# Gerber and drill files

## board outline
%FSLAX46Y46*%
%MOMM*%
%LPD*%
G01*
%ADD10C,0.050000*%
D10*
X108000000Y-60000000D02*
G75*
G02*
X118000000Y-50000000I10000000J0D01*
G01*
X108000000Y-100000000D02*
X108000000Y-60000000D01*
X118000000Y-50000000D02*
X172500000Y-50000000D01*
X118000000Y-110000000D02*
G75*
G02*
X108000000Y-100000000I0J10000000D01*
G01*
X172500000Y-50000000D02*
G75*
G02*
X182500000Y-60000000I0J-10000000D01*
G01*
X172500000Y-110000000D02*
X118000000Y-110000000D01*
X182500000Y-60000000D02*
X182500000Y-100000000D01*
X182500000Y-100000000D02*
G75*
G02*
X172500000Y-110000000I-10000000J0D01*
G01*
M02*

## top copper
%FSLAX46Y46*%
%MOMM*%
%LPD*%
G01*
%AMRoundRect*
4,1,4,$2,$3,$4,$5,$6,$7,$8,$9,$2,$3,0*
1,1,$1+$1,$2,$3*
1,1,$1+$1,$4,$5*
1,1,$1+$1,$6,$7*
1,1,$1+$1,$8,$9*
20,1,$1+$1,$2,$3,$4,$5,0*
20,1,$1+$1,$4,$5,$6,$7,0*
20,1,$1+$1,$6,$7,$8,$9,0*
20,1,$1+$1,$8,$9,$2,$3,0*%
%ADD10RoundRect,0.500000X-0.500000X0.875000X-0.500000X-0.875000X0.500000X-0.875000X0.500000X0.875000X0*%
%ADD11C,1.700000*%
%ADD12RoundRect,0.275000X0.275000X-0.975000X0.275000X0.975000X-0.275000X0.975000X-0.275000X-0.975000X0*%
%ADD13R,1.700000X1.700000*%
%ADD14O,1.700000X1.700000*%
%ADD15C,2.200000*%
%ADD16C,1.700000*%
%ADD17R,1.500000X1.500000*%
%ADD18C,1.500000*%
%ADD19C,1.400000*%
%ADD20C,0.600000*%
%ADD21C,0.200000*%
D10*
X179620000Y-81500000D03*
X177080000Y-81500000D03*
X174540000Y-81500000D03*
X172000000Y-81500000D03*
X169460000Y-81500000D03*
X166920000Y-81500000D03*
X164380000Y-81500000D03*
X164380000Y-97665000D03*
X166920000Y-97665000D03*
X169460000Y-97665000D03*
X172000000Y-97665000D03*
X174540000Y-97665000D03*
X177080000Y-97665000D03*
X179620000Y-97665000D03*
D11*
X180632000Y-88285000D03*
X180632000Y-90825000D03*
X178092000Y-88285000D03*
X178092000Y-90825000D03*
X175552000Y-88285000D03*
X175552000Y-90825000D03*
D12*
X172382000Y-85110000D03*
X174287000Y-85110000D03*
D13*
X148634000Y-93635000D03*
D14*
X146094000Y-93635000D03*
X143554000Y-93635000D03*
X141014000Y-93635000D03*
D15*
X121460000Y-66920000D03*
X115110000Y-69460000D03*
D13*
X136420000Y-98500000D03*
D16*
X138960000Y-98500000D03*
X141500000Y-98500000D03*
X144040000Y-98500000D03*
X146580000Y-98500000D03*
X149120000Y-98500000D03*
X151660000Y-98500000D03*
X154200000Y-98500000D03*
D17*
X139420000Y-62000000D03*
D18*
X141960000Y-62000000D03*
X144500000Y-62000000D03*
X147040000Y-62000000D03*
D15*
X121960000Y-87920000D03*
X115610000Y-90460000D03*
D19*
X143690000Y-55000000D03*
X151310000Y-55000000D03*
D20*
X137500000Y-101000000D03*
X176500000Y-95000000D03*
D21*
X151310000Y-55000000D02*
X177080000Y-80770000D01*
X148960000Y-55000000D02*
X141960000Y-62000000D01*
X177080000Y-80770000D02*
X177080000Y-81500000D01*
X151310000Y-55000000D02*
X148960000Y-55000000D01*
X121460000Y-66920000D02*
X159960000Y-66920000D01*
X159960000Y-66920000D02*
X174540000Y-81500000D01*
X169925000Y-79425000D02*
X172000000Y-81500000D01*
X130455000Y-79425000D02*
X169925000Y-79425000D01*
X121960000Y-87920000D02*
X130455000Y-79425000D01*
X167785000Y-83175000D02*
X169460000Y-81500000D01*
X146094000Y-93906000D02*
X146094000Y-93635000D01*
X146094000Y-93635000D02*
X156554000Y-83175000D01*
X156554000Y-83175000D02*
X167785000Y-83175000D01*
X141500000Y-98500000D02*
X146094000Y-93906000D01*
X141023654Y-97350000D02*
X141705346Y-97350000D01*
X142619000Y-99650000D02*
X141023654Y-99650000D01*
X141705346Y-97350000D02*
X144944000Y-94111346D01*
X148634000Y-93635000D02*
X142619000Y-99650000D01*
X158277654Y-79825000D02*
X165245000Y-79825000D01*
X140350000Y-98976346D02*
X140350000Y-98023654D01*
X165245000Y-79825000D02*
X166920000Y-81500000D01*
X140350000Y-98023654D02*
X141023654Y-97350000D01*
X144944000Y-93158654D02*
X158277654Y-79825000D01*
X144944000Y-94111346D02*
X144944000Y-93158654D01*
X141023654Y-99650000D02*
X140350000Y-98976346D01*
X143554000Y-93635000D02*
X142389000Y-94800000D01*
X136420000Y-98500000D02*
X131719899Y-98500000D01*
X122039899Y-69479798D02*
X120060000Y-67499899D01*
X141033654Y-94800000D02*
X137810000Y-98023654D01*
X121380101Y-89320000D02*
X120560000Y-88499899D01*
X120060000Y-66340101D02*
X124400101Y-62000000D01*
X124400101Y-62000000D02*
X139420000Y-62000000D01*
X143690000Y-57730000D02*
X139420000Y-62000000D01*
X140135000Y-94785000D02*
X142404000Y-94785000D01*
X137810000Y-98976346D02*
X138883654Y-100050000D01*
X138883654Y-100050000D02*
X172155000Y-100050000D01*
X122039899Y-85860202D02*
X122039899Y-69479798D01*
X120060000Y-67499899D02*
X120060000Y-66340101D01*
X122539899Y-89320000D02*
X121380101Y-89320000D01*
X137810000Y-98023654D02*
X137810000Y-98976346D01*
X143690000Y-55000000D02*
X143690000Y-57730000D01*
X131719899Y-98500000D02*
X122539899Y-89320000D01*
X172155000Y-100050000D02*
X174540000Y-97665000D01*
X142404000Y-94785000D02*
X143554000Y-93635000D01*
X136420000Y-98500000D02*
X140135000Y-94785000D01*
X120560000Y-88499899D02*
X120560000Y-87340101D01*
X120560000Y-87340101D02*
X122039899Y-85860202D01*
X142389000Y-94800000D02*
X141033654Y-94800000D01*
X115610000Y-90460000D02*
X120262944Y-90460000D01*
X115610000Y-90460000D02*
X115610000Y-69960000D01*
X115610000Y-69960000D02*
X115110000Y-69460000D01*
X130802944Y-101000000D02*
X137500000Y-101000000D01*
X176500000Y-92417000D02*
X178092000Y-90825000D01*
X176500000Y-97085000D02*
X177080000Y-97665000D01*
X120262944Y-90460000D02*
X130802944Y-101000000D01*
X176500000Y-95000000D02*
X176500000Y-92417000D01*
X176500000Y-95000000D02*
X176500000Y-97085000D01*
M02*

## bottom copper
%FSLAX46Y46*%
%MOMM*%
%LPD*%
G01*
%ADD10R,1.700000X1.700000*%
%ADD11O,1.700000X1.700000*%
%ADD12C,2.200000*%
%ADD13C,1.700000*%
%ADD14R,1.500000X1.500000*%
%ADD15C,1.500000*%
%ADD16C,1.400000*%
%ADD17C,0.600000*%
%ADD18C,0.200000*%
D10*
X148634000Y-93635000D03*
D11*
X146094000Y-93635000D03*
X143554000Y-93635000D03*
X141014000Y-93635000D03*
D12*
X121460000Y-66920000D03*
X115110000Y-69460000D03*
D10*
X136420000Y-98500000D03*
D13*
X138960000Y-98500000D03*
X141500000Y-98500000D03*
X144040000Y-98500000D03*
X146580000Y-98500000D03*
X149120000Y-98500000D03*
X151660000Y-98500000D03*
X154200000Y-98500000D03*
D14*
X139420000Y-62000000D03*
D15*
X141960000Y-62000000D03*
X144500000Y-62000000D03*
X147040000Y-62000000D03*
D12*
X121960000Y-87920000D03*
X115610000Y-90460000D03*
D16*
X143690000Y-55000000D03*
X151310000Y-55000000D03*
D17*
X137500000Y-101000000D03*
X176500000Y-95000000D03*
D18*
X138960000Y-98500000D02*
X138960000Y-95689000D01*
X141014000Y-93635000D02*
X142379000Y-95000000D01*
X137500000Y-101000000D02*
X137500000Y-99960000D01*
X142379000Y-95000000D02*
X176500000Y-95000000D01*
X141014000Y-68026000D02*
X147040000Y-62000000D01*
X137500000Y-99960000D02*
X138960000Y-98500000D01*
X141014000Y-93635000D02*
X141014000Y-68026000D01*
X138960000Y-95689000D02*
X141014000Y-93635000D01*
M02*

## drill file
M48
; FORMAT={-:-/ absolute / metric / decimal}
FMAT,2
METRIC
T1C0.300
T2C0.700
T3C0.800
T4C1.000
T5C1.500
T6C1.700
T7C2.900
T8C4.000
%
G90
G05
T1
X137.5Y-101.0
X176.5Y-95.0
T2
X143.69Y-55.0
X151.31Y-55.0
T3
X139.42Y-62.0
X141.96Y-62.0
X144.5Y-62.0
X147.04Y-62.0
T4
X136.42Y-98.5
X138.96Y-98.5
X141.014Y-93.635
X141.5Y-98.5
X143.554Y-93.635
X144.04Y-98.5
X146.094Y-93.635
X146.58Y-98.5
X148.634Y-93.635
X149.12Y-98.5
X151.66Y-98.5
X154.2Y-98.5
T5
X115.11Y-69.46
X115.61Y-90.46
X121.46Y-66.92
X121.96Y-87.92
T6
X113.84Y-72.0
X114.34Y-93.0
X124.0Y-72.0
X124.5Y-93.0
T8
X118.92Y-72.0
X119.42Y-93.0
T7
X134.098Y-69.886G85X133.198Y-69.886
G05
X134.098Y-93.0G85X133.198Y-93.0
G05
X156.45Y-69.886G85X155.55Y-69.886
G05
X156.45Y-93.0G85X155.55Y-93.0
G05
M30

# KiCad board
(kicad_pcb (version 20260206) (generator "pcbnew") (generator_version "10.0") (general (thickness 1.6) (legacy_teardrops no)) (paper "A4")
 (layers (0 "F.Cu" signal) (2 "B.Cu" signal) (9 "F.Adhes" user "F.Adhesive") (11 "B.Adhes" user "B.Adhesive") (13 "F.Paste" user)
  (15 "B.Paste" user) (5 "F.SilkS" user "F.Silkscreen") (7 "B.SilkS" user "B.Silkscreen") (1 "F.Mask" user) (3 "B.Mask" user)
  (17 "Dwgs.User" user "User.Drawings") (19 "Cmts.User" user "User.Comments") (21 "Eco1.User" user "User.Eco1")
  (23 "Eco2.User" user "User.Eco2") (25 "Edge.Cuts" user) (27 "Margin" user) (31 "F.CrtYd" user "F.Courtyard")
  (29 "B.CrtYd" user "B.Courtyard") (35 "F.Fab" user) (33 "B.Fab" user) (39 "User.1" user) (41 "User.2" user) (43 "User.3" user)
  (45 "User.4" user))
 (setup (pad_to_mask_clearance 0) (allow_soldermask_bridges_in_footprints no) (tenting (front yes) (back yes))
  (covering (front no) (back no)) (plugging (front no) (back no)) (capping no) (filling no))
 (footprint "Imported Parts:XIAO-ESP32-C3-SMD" (layer "F.Cu") (at 161.5 80.665 -90)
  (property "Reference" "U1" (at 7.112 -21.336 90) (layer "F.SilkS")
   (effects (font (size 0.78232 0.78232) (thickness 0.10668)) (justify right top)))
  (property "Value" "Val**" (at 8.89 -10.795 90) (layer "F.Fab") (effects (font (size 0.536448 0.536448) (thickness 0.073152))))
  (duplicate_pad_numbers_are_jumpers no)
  (pad "1" smd roundrect (at 0.835 -18.12 270) (size 2.75 2) (layers "F.Cu" "F.Mask" "F.Paste") (roundrect_rratio 0.25)
   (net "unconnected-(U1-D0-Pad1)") (solder_mask_margin 0.0508) (thermal_bridge_angle 45))
  (pad "2" smd roundrect (at 0.835 -15.58 270) (size 2.75 2) (layers "F.Cu" "F.Mask" "F.Paste") (roundrect_rratio 0.25) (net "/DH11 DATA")
   (solder_mask_margin 0.0508) (thermal_bridge_angle 45))
  (pad "3" smd roundrect (at 0.835 -13.04 270) (size 2.75 2) (layers "F.Cu" "F.Mask" "F.Paste") (roundrect_rratio 0.25) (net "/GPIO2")
   (solder_mask_margin 0.0508) (thermal_bridge_angle 45))
  (pad "4" smd roundrect (at 0.835 -10.5 270) (size 2.75 2) (layers "F.Cu" "F.Mask" "F.Paste") (roundrect_rratio 0.25) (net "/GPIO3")
   (solder_mask_margin 0.0508) (thermal_bridge_angle 45))
  (pad "5" smd roundrect (at 0.835 -7.96 270) (size 2.75 2) (layers "F.Cu" "F.Mask" "F.Paste") (roundrect_rratio 0.25) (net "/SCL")
   (solder_mask_margin 0.0508) (thermal_bridge_angle 45))
  (pad "6" smd roundrect (at 0.835 -5.42 270) (size 2.75 2) (layers "F.Cu" "F.Mask" "F.Paste") (roundrect_rratio 0.25) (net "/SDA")
   (solder_mask_margin 0.0508) (thermal_bridge_angle 45))
  (pad "7" smd roundrect (at 0.835 -2.88 270) (size 2.75 2) (layers "F.Cu" "F.Mask" "F.Paste") (roundrect_rratio 0.25)
   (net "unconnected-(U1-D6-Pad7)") (solder_mask_margin 0.0508) (thermal_bridge_angle 45))
  (pad "8" smd roundrect (at 17 -2.88 270) (size 2.75 2) (layers "F.Cu" "F.Mask" "F.Paste") (roundrect_rratio 0.25)
   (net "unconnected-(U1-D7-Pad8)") (solder_mask_margin 0.0508) (thermal_bridge_angle 45))
  (pad "9" smd roundrect (at 17 -5.42 270) (size 2.75 2) (layers "F.Cu" "F.Mask" "F.Paste") (roundrect_rratio 0.25)
   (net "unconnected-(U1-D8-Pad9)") (solder_mask_margin 0.0508) (thermal_bridge_angle 45))
  (pad "10" smd roundrect (at 17 -7.96 270) (size 2.75 2) (layers "F.Cu" "F.Mask" "F.Paste") (roundrect_rratio 0.25)
   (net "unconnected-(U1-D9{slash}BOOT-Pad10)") (solder_mask_margin 0.0508) (thermal_bridge_angle 45))
  (pad "11" smd roundrect (at 17 -10.5 270) (size 2.75 2) (layers "F.Cu" "F.Mask" "F.Paste") (roundrect_rratio 0.25)
   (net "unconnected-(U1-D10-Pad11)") (solder_mask_margin 0.0508) (thermal_bridge_angle 45))
  (pad "12" smd roundrect (at 17 -13.04 270) (size 2.75 2) (layers "F.Cu" "F.Mask" "F.Paste") (roundrect_rratio 0.25) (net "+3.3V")
   (solder_mask_margin 0.0508) (thermal_bridge_angle 45))
  (pad "13" smd roundrect (at 17 -15.58 270) (size 2.75 2) (layers "F.Cu" "F.Mask" "F.Paste") (roundrect_rratio 0.25) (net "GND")
   (solder_mask_margin 0.0508) (thermal_bridge_angle 45))
  (pad "14" smd roundrect (at 17 -18.12 270) (size 2.75 2) (layers "F.Cu" "F.Mask" "F.Paste") (roundrect_rratio 0.25) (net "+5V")
   (solder_mask_margin 0.0508) (thermal_bridge_angle 45))
  (pad "15" smd circle (at 7.62 -19.132 270) (size 1.7 1.7) (layers "F.Cu" "F.Mask" "F.Paste") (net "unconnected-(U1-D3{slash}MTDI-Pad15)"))
  (pad "16" smd circle (at 10.16 -19.132 270) (size 1.7 1.7) (layers "F.Cu" "F.Mask" "F.Paste") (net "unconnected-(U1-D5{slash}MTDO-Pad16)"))
  (pad "17" smd circle (at 7.62 -16.592 270) (size 1.7 1.7) (layers "F.Cu" "F.Mask" "F.Paste") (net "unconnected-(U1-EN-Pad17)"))
  (pad "18" smd circle (at 10.16 -16.592 270) (size 1.7 1.7) (layers "F.Cu" "F.Mask" "F.Paste") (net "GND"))
  (pad "19" smd circle (at 7.62 -14.052 270) (size 1.7 1.7) (layers "F.Cu" "F.Mask" "F.Paste") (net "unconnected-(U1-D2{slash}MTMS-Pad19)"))
  (pad "20" smd circle (at 10.16 -14.052 270) (size 1.7 1.7) (layers "F.Cu" "F.Mask" "F.Paste") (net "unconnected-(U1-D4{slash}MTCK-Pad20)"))
  (pad "21" smd roundrect (at 4.445 -10.882 90) (size 2.5 1.1) (layers "F.Cu" "F.Mask" "F.Paste") (roundrect_rratio 0.25)
   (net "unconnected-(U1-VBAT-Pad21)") (thermal_bridge_angle 45))
  (pad "22" smd roundrect (at 4.445 -12.787 90) (size 2.5 1.1) (layers "F.Cu" "F.Mask" "F.Paste") (roundrect_rratio 0.25)
   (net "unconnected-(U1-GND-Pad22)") (thermal_bridge_angle 45)))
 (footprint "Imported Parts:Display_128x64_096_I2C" (layer "F.Cu") (at 144.824 93.635 180)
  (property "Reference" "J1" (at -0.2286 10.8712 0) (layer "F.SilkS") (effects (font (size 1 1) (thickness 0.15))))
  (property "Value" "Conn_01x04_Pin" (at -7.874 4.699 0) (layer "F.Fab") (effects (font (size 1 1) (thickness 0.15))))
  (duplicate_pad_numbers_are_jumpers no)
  (pad "" np_thru_hole oval (at -11.176 0.635 180) (size 3.8 2.9) (drill oval 3.8 2.9) (layers "*.Cu" "*.Mask"))
  (pad "" np_thru_hole oval (at -11.176 23.749 180) (size 3.8 2.9) (drill oval 3.8 2.9) (layers "*.Cu" "*.Mask"))
  (pad "" np_thru_hole oval (at 11.176 0.635 180) (size 3.8 2.9) (drill oval 3.8 2.9) (layers "*.Cu" "*.Mask"))
  (pad "" np_thru_hole oval (at 11.176 23.749 180) (size 3.8 2.9) (drill oval 3.8 2.9) (layers "*.Cu" "*.Mask"))
  (pad "1" thru_hole rect (at -3.81 0 270) (size 1.7 1.7) (drill 1) (layers "*.Cu" "*.Mask") (remove_unused_layers no) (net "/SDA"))
  (pad "2" thru_hole oval (at -1.27 0 270) (size 1.7 1.7) (drill 1) (layers "*.Cu" "*.Mask") (remove_unused_layers no) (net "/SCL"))
  (pad "3" thru_hole oval (at 1.27 0 270) (size 1.7 1.7) (drill 1) (layers "*.Cu" "*.Mask") (remove_unused_layers no) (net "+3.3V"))
  (pad "4" thru_hole oval (at 3.81 0 270) (size 1.7 1.7) (drill 1) (layers "*.Cu" "*.Mask") (remove_unused_layers no) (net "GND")))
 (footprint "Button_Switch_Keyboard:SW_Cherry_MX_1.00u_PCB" (layer "F.Cu") (at 121.46 66.92)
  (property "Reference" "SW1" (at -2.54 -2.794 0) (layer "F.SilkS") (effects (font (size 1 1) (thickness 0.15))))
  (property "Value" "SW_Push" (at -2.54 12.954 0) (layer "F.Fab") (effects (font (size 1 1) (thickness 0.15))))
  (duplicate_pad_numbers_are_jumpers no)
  (pad "" np_thru_hole circle (at -7.62 5.08) (size 1.7 1.7) (drill 1.7) (layers "*.Cu" "*.Mask"))
  (pad "" np_thru_hole circle (at -2.54 5.08) (size 4 4) (drill 4) (layers "*.Cu" "*.Mask"))
  (pad "" np_thru_hole circle (at 2.54 5.08) (size 1.7 1.7) (drill 1.7) (layers "*.Cu" "*.Mask"))
  (pad "1" thru_hole circle (at 0 0) (size 2.2 2.2) (drill 1.5) (layers "*.Cu" "*.Mask") (remove_unused_layers no) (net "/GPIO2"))
  (pad "2" thru_hole circle (at -6.35 2.54) (size 2.2 2.2) (drill 1.5) (layers "*.Cu" "*.Mask") (remove_unused_layers no) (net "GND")))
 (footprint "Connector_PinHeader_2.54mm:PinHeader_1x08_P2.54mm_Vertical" (layer "F.Cu") (at 136.42 98.5 90)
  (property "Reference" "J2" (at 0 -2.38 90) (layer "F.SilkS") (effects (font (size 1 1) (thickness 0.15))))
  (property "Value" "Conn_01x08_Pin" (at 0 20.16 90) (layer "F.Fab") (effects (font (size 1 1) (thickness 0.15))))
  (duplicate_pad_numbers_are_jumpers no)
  (pad "1" thru_hole rect (at 0 0 90) (size 1.7 1.7) (drill 1) (layers "*.Cu" "*.Mask") (remove_unused_layers no) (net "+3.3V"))
  (pad "2" thru_hole circle (at 0 2.54 90) (size 1.7 1.7) (drill 1) (layers "*.Cu" "*.Mask") (remove_unused_layers no) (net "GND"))
  (pad "3" thru_hole circle (at 0 5.08 90) (size 1.7 1.7) (drill 1) (layers "*.Cu" "*.Mask") (remove_unused_layers no) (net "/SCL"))
  (pad "4" thru_hole circle (at 0 7.62 90) (size 1.7 1.7) (drill 1) (layers "*.Cu" "*.Mask") (remove_unused_layers no) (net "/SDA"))
  (pad "5" thru_hole circle (at 0 10.16 90) (size 1.7 1.7) (drill 1) (layers "*.Cu" "*.Mask") (remove_unused_layers no)
   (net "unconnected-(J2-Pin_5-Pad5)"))
  (pad "6" thru_hole circle (at 0 12.7 90) (size 1.7 1.7) (drill 1) (layers "*.Cu" "*.Mask") (remove_unused_layers no)
   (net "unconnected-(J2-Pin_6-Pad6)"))
  (pad "7" thru_hole circle (at 0 15.24 90) (size 1.7 1.7) (drill 1) (layers "*.Cu" "*.Mask") (remove_unused_layers no)
   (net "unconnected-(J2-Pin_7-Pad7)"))
  (pad "8" thru_hole circle (at 0 17.78 90) (size 1.7 1.7) (drill 1) (layers "*.Cu" "*.Mask") (remove_unused_layers no)
   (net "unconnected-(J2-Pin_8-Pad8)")))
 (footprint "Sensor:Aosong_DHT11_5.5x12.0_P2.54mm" (layer "F.Cu") (at 139.42 62 90)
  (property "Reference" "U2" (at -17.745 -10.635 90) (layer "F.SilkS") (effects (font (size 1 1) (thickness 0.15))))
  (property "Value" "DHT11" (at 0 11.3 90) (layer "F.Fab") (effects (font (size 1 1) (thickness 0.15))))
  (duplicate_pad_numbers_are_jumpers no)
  (pad "1" thru_hole rect (at 0 0 90) (size 1.5 1.5) (drill 0.8) (layers "*.Cu" "*.Mask") (remove_unused_layers no) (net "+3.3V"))
  (pad "2" thru_hole circle (at 0 2.54 90) (size 1.5 1.5) (drill 0.8) (layers "*.Cu" "*.Mask") (remove_unused_layers no) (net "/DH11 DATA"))
  (pad "3" thru_hole circle (at 0 5.08 90) (size 1.5 1.5) (drill 0.8) (layers "*.Cu" "*.Mask") (remove_unused_layers no)
   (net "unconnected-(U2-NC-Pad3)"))
  (pad "4" thru_hole circle (at 0 7.62 90) (size 1.5 1.5) (drill 0.8) (layers "*.Cu" "*.Mask") (remove_unused_layers no) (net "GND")))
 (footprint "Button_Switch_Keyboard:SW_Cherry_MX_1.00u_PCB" (layer "F.Cu") (at 121.96 87.92)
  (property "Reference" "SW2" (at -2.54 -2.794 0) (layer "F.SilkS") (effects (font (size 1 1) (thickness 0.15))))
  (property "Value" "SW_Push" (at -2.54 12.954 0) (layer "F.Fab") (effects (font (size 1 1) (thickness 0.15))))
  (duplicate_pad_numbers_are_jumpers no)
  (pad "" np_thru_hole circle (at -7.62 5.08) (size 1.7 1.7) (drill 1.7) (layers "*.Cu" "*.Mask"))
  (pad "" np_thru_hole circle (at -2.54 5.08) (size 4 4) (drill 4) (layers "*.Cu" "*.Mask"))
  (pad "" np_thru_hole circle (at 2.54 5.08) (size 1.7 1.7) (drill 1.7) (layers "*.Cu" "*.Mask"))
  (pad "1" thru_hole circle (at 0 0) (size 2.2 2.2) (drill 1.5) (layers "*.Cu" "*.Mask") (remove_unused_layers no) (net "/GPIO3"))
  (pad "2" thru_hole circle (at -6.35 2.54) (size 2.2 2.2) (drill 1.5) (layers "*.Cu" "*.Mask") (remove_unused_layers no) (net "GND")))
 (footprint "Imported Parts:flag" (layer "F.Cu") (at 120.5 56)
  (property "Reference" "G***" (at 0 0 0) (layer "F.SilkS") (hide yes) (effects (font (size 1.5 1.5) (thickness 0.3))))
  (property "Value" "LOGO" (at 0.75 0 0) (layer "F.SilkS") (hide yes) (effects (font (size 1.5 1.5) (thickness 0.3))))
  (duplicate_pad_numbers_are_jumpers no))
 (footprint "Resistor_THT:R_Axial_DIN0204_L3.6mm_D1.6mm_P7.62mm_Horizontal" (layer "F.Cu") (at 143.69 55)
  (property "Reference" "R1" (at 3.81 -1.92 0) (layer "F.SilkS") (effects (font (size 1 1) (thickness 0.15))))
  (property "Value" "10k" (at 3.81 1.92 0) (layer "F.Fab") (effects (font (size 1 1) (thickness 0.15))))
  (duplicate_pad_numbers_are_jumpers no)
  (pad "1" thru_hole circle (at 0 0) (size 1.4 1.4) (drill 0.7) (layers "*.Cu" "*.Mask") (remove_unused_layers no) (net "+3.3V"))
  (pad "2" thru_hole circle (at 7.62 0) (size 1.4 1.4) (drill 0.7) (layers "*.Cu" "*.Mask") (remove_unused_layers no) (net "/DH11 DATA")))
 (gr_arc (start 108 60) (mid 110.928932 52.928932) (end 118 50) (stroke (width 0.05) (type default)) (layer "Edge.Cuts"))
 (gr_line (start 108 100) (end 108 60) (stroke (width 0.05) (type default)) (layer "Edge.Cuts"))
 (gr_line (start 118 50) (end 172.5 50) (stroke (width 0.05) (type default)) (layer "Edge.Cuts"))
 (gr_arc (start 118 110) (mid 110.928932 107.071068) (end 108 100) (stroke (width 0.05) (type default)) (layer "Edge.Cuts"))
 (gr_arc (start 172.5 50) (mid 179.571068 52.928932) (end 182.5 60) (stroke (width 0.05) (type default)) (layer "Edge.Cuts"))
 (gr_line (start 172.5 110) (end 118 110) (stroke (width 0.05) (type default)) (layer "Edge.Cuts"))
 (gr_line (start 182.5 60) (end 182.5 100) (stroke (width 0.05) (type default)) (layer "Edge.Cuts"))
 (gr_arc (start 182.5 100) (mid 179.571068 107.071068) (end 172.5 110) (stroke (width 0.05) (type default)) (layer "Edge.Cuts"))
 (segment (start 151.31 55) (end 177.08 80.77) (width 0.2) (layer "F.Cu") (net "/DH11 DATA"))
 (segment (start 148.96 55) (end 141.96 62) (width 0.2) (layer "F.Cu") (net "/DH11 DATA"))
 (segment (start 177.08 80.77) (end 177.08 81.5) (width 0.2) (layer "F.Cu") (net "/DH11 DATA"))
 (segment (start 151.31 55) (end 148.96 55) (width 0.2) (layer "F.Cu") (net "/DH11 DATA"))
 (segment (start 121.46 66.92) (end 159.96 66.92) (width 0.2) (layer "F.Cu") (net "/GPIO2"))
 (segment (start 159.96 66.92) (end 174.54 81.5) (width 0.2) (layer "F.Cu") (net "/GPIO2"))
 (segment (start 169.925 79.425) (end 172 81.5) (width 0.2) (layer "F.Cu") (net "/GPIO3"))
 (segment (start 130.455 79.425) (end 169.925 79.425) (width 0.2) (layer "F.Cu") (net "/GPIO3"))
 (segment (start 121.96 87.92) (end 130.455 79.425) (width 0.2) (layer "F.Cu") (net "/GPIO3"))
 (segment (start 167.785 83.175) (end 169.46 81.5) (width 0.2) (layer "F.Cu") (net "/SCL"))
 (segment (start 146.094 93.906) (end 146.094 93.635) (width 0.2) (layer "F.Cu") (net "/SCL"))
 (segment (start 146.094 93.635) (end 156.554 83.175) (width 0.2) (layer "F.Cu") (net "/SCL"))
 (segment (start 156.554 83.175) (end 167.785 83.175) (width 0.2) (layer "F.Cu") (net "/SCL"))
 (segment (start 141.5 98.5) (end 146.094 93.906) (width 0.2) (layer "F.Cu") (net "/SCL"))
 (segment (start 141.023654 97.35) (end 141.705346 97.35) (width 0.2) (layer "F.Cu") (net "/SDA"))
 (segment (start 142.619 99.65) (end 141.023654 99.65) (width 0.2) (layer "F.Cu") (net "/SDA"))
 (segment (start 141.705346 97.35) (end 144.944 94.111346) (width 0.2) (layer "F.Cu") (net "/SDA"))
 (segment (start 148.634 93.635) (end 142.619 99.65) (width 0.2) (layer "F.Cu") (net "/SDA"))
 (segment (start 158.277654 79.825) (end 165.245 79.825) (width 0.2) (layer "F.Cu") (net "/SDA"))
 (segment (start 140.35 98.976346) (end 140.35 98.023654) (width 0.2) (layer "F.Cu") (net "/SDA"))
 (segment (start 165.245 79.825) (end 166.92 81.5) (width 0.2) (layer "F.Cu") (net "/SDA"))
 (segment (start 140.35 98.023654) (end 141.023654 97.35) (width 0.2) (layer "F.Cu") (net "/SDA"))
 (segment (start 144.944 93.158654) (end 158.277654 79.825) (width 0.2) (layer "F.Cu") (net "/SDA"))
 (segment (start 144.944 94.111346) (end 144.944 93.158654) (width 0.2) (layer "F.Cu") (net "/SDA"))
 (segment (start 141.023654 99.65) (end 140.35 98.976346) (width 0.2) (layer "F.Cu") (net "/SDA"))
 (segment (start 143.554 93.635) (end 142.389 94.8) (width 0.2) (layer "F.Cu") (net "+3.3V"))
 (segment (start 136.42 98.5) (end 131.719899 98.5) (width 0.2) (layer "F.Cu") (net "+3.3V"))
 (segment (start 122.039899 69.479798) (end 120.06 67.499899) (width 0.2) (layer "F.Cu") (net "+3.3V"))
 (segment (start 141.033654 94.8) (end 137.81 98.023654) (width 0.2) (layer "F.Cu") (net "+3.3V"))
 (segment (start 121.380101 89.32) (end 120.56 88.499899) (width 0.2) (layer "F.Cu") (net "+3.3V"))
 (segment (start 120.06 66.340101) (end 124.400101 62) (width 0.2) (layer "F.Cu") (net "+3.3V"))
 (segment (start 124.400101 62) (end 139.42 62) (width 0.2) (layer "F.Cu") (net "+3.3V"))
 (segment (start 143.69 57.73) (end 139.42 62) (width 0.2) (layer "F.Cu") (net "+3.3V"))
 (segment (start 140.135 94.785) (end 142.404 94.785) (width 0.2) (layer "F.Cu") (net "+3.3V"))
 (segment (start 137.81 98.976346) (end 138.883654 100.05) (width 0.2) (layer "F.Cu") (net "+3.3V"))
 (segment (start 138.883654 100.05) (end 172.155 100.05) (width 0.2) (layer "F.Cu") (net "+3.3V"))
 (segment (start 122.039899 85.860202) (end 122.039899 69.479798) (width 0.2) (layer "F.Cu") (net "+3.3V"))
 (segment (start 120.06 67.499899) (end 120.06 66.340101) (width 0.2) (layer "F.Cu") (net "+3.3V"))
 (segment (start 122.539899 89.32) (end 121.380101 89.32) (width 0.2) (layer "F.Cu") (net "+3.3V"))
 (segment (start 137.81 98.023654) (end 137.81 98.976346) (width 0.2) (layer "F.Cu") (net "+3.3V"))
 (segment (start 143.69 55) (end 143.69 57.73) (width 0.2) (layer "F.Cu") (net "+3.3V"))
 (segment (start 131.719899 98.5) (end 122.539899 89.32) (width 0.2) (layer "F.Cu") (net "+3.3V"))
 (segment (start 172.155 100.05) (end 174.54 97.665) (width 0.2) (layer "F.Cu") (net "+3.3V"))
 (segment (start 142.404 94.785) (end 143.554 93.635) (width 0.2) (layer "F.Cu") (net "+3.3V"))
 (segment (start 136.42 98.5) (end 140.135 94.785) (width 0.2) (layer "F.Cu") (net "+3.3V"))
 (segment (start 120.56 88.499899) (end 120.56 87.340101) (width 0.2) (layer "F.Cu") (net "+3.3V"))
 (segment (start 120.56 87.340101) (end 122.039899 85.860202) (width 0.2) (layer "F.Cu") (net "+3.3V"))
 (segment (start 142.389 94.8) (end 141.033654 94.8) (width 0.2) (layer "F.Cu") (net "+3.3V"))
 (segment (start 115.61 90.46) (end 120.262944 90.46) (width 0.2) (layer "F.Cu") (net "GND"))
 (segment (start 115.61 90.46) (end 115.61 69.96) (width 0.2) (layer "F.Cu") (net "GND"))
 (segment (start 115.61 69.96) (end 115.11 69.46) (width 0.2) (layer "F.Cu") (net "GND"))
 (segment (start 130.802944 101) (end 137.5 101) (width 0.2) (layer "F.Cu") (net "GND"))
 (segment (start 176.5 92.417) (end 178.092 90.825) (width 0.2) (layer "F.Cu") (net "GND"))
 (segment (start 176.5 97.085) (end 177.08 97.665) (width 0.2) (layer "F.Cu") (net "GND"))
 (segment (start 120.262944 90.46) (end 130.802944 101) (width 0.2) (layer "F.Cu") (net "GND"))
 (segment (start 176.5 95) (end 176.5 92.417) (width 0.2) (layer "F.Cu") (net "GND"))
 (segment (start 176.5 95) (end 176.5 97.085) (width 0.2) (layer "F.Cu") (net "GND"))
 (via (at 137.5 101) (size 0.6) (drill 0.3) (layers "F.Cu" "B.Cu") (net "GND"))
 (via (at 176.5 95) (size 0.6) (drill 0.3) (layers "F.Cu" "B.Cu") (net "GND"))
 (segment (start 138.96 98.5) (end 138.96 95.689) (width 0.2) (layer "B.Cu") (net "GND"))
 (segment (start 141.014 93.635) (end 142.379 95) (width 0.2) (layer "B.Cu") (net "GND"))
 (segment (start 137.5 101) (end 137.5 99.96) (width 0.2) (layer "B.Cu") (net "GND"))
 (segment (start 142.379 95) (end 176.5 95) (width 0.2) (layer "B.Cu") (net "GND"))
 (segment (start 141.014 68.026) (end 147.04 62) (width 0.2) (layer "B.Cu") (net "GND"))
 (segment (start 137.5 99.96) (end 138.96 98.5) (width 0.2) (layer "B.Cu") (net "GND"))
 (segment (start 141.014 93.635) (end 141.014 68.026) (width 0.2) (layer "B.Cu") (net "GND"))
 (segment (start 138.96 95.689) (end 141.014 93.635) (width 0.2) (layer "B.Cu") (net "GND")))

